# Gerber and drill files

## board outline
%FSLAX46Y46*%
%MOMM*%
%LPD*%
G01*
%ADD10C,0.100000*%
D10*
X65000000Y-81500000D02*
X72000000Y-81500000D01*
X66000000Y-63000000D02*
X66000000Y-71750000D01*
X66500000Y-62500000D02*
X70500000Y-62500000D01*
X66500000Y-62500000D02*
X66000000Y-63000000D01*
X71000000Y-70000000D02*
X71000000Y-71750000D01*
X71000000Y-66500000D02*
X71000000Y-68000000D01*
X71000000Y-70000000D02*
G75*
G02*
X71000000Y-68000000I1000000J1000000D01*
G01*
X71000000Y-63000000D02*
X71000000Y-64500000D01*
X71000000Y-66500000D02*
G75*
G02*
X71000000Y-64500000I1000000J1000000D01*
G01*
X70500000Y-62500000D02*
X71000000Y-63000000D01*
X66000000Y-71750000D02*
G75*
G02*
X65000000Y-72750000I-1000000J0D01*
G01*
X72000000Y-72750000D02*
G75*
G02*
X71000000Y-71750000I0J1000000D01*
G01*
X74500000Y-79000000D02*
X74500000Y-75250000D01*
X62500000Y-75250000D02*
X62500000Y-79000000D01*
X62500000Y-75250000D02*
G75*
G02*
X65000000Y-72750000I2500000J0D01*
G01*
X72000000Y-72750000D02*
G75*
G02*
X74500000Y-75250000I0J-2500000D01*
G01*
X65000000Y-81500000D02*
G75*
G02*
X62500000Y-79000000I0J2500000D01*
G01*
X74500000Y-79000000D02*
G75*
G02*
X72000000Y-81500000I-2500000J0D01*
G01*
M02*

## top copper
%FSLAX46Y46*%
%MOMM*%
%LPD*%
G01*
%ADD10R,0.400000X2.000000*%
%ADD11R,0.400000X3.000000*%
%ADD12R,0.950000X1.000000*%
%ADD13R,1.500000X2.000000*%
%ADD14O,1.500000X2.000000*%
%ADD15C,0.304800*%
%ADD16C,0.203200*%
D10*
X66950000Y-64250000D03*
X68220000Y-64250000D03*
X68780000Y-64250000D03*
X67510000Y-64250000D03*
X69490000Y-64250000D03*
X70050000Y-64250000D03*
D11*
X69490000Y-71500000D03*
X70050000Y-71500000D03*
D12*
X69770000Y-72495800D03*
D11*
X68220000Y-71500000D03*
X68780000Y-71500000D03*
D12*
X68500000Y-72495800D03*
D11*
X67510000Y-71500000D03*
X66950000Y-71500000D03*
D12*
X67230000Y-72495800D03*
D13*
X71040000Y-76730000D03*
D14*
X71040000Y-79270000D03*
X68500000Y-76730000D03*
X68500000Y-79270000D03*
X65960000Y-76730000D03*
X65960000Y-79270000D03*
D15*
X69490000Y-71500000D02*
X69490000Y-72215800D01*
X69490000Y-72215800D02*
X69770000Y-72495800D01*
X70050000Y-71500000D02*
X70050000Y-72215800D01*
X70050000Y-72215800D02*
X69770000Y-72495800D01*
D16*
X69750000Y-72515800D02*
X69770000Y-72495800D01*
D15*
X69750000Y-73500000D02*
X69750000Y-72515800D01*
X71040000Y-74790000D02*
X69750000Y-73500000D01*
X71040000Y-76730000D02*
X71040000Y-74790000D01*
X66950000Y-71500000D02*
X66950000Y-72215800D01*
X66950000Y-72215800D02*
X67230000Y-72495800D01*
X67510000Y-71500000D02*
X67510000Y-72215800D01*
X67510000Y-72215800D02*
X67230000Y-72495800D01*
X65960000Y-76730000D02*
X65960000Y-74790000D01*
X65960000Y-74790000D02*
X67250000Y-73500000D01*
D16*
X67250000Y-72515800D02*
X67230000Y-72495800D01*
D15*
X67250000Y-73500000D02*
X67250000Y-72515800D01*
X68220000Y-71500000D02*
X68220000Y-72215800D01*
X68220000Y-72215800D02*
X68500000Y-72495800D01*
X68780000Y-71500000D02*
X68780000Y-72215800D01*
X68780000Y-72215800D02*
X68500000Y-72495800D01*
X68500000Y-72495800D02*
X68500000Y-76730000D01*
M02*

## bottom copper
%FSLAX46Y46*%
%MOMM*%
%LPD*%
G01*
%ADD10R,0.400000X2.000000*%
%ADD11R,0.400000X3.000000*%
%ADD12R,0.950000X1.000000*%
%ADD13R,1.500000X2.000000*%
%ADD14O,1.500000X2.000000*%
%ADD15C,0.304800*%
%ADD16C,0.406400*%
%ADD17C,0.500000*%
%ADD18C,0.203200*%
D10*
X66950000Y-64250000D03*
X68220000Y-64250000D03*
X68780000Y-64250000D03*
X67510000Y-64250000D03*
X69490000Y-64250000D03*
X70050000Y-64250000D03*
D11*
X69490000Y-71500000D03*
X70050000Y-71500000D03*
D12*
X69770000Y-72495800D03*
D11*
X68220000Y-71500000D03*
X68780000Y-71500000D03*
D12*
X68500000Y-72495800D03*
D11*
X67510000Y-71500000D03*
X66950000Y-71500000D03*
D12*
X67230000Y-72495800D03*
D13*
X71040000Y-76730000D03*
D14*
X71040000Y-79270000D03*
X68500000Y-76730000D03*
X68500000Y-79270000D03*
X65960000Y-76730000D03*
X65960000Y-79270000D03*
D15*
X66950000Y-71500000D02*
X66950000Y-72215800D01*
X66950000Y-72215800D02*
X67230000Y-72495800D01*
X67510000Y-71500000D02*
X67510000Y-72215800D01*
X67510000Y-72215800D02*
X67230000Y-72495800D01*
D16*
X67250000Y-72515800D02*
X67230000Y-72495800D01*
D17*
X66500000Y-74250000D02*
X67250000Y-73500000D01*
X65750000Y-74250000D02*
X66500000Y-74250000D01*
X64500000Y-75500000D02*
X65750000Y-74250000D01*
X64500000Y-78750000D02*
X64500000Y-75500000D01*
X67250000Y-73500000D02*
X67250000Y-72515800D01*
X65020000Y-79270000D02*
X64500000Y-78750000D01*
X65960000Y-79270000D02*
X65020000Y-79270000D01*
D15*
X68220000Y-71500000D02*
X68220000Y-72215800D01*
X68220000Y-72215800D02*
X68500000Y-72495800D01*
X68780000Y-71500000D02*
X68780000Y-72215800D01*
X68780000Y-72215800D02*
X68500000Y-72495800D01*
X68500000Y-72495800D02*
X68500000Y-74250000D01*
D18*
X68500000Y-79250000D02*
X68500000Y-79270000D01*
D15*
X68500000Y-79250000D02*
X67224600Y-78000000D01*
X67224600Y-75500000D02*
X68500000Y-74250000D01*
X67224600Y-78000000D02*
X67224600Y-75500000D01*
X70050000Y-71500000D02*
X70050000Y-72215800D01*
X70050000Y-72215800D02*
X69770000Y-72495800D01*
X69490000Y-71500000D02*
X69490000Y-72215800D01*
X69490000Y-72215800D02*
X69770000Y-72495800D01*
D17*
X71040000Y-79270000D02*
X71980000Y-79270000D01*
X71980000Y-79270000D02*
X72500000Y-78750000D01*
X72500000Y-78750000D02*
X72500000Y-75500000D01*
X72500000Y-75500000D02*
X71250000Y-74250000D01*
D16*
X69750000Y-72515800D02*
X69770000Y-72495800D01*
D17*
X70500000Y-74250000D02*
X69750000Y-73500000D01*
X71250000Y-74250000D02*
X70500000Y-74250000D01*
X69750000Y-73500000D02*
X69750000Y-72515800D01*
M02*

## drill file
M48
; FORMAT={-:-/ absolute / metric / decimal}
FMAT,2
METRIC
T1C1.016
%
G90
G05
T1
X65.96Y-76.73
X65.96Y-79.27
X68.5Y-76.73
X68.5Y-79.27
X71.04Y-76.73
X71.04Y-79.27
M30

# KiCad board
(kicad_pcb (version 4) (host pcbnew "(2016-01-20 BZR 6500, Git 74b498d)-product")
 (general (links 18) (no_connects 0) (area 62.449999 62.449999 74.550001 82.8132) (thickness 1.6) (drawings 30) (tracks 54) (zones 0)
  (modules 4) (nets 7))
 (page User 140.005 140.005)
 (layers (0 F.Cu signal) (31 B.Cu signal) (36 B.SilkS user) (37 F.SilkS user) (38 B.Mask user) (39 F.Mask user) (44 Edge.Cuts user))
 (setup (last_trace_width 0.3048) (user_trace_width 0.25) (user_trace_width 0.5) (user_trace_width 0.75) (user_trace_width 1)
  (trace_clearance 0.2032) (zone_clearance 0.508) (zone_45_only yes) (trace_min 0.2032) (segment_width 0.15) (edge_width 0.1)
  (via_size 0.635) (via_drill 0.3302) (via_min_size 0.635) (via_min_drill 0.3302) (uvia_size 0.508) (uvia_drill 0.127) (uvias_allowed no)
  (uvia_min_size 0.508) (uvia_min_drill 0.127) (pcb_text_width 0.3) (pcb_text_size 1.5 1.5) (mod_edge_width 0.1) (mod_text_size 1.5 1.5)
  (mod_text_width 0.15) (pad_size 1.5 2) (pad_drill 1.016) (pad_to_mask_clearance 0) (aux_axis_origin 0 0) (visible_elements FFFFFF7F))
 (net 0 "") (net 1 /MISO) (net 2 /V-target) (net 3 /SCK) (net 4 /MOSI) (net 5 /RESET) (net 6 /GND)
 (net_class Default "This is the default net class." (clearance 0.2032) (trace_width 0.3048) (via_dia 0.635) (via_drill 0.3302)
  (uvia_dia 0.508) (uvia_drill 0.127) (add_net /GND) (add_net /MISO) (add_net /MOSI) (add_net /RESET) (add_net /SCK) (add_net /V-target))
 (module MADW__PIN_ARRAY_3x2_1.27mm (layer F.Cu) (at 68.5 68) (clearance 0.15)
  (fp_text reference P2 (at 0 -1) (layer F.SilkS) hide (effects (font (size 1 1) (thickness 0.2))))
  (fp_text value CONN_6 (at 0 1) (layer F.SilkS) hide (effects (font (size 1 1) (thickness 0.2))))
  (pad ~ smd rect (at -1.55 -3.75) (size 0.4 2) (layers F.Cu F.Mask))
  (pad ~ smd rect (at -0.28 -3.75) (size 0.4 2) (layers F.Cu F.Mask))
  (pad ~ smd rect (at 0.28 -3.75) (size 0.4 2) (layers F.Cu F.Mask))
  (pad ~ smd rect (at -0.99 -3.75) (size 0.4 2) (layers F.Cu F.Mask))
  (pad ~ smd rect (at 0.99 -3.75) (size 0.4 2) (layers F.Cu F.Mask))
  (pad ~ smd rect (at 1.55 -3.75) (size 0.4 2) (layers F.Cu F.Mask))
  (pad ~ smd rect (at -1.55 -3.75) (size 0.4 2) (layers B.Cu F.Mask))
  (pad ~ smd rect (at -0.28 -3.75) (size 0.4 2) (layers B.Cu F.Mask))
  (pad ~ smd rect (at 0.28 -3.75) (size 0.4 2) (layers B.Cu F.Mask))
  (pad ~ smd rect (at -0.99 -3.75) (size 0.4 2) (layers B.Cu F.Mask))
  (pad ~ smd rect (at 0.99 -3.75) (size 0.4 2) (layers B.Cu F.Mask))
  (pad ~ smd rect (at 1.55 -3.75) (size 0.4 2) (layers B.Cu F.Mask))
  (pad 1 smd rect (at 0.99 3.5) (size 0.4 3) (layers F.Cu F.Mask) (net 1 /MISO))
  (pad 1 smd rect (at 1.55 3.5) (size 0.4 3) (layers F.Cu F.Mask) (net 1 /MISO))
  (pad 1 smd rect (at 1.27 4.4958) (size 0.95 1) (layers F.Cu F.Mask) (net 1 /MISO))
  (pad 2 smd rect (at 0.99 3.5) (size 0.4 3) (layers B.Cu F.Mask) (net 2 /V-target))
  (pad 2 smd rect (at 1.55 3.5) (size 0.4 3) (layers B.Cu F.Mask) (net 2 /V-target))
  (pad 2 smd rect (at 1.27 4.4958) (size 0.95 1) (layers B.Cu B.Mask) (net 2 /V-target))
  (pad 3 smd rect (at -0.28 3.5) (size 0.4 3) (layers F.Cu F.Mask) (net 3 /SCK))
  (pad 3 smd rect (at 0.28 3.5) (size 0.4 3) (layers F.Cu F.Mask) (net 3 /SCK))
  (pad 3 smd rect (at 0 4.4958) (size 0.95 1) (layers F.Cu F.Mask) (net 3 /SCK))
  (pad 4 smd rect (at -0.28 3.5) (size 0.4 3) (layers B.Cu F.Mask) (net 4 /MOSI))
  (pad 4 smd rect (at 0.28 3.5) (size 0.4 3) (layers B.Cu F.Mask) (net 4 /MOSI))
  (pad 4 smd rect (at 0 4.4958) (size 0.95 1) (layers B.Cu B.Mask) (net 4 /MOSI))
  (pad 5 smd rect (at -0.99 3.5) (size 0.4 3) (layers F.Cu F.Mask) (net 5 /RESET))
  (pad 5 smd rect (at -1.55 3.5) (size 0.4 3) (layers F.Cu F.Mask) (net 5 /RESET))
  (pad 5 smd rect (at -1.27 4.4958) (size 0.95 1) (layers F.Cu F.Mask) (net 5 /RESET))
  (pad 6 smd rect (at -0.99 3.5) (size 0.4 3) (layers B.Cu F.Mask) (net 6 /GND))
  (pad 6 smd rect (at -1.55 3.5) (size 0.4 3) (layers B.Cu F.Mask) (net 6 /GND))
  (pad 6 smd rect (at -1.27 4.4958) (size 0.95 1) (layers B.Cu B.Mask) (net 6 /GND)))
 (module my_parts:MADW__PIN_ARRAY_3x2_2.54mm (layer F.Cu) (at 68.5 78)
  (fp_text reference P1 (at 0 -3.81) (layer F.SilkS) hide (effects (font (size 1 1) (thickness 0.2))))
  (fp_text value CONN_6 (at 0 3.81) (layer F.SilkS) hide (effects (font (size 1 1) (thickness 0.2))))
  (pad 1 thru_hole rect (at 2.54 -1.27) (size 1.5 2) (drill 1.016) (layers *.Cu *.Mask F.SilkS) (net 1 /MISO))
  (pad 2 thru_hole oval (at 2.54 1.27) (size 1.5 2) (drill 1.016) (layers *.Cu *.Mask F.SilkS) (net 2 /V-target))
  (pad 3 thru_hole oval (at 0 -1.27) (size 1.5 2) (drill 1.016) (layers *.Cu *.Mask F.SilkS) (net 3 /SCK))
  (pad 4 thru_hole oval (at 0 1.27) (size 1.5 2) (drill 1.016) (layers *.Cu *.Mask F.SilkS) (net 4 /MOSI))
  (pad 5 thru_hole oval (at -2.54 -1.27) (size 1.5 2) (drill 1.016) (layers *.Cu *.Mask F.SilkS) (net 5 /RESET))
  (pad 6 thru_hole oval (at -2.54 1.27) (size 1.5 2) (drill 1.016) (layers *.Cu *.Mask F.SilkS) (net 6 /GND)))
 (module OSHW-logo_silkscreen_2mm (layer F.Cu) (at 71.95 74.2)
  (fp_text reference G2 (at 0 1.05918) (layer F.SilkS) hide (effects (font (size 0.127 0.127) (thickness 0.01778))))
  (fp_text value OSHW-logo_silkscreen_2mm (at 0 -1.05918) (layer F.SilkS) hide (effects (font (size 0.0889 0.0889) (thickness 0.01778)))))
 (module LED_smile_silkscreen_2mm (layer F.Cu) (at 64.75 74.25)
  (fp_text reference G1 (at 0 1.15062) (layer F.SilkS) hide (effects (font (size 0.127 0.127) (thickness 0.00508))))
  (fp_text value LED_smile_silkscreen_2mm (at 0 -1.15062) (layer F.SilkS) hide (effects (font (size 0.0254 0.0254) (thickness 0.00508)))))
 (gr_line (start 65 81.5) (end 72 81.5) (layer Edge.Cuts) (width 0.1))
 (gr_line (start 66 63) (end 66 71.75) (angle 90) (layer Edge.Cuts) (width 0.1))
 (gr_line (start 66.5 62.5) (end 70.5 62.5) (angle 90) (layer Edge.Cuts) (width 0.1))
 (gr_line (start 66.5 62.5) (end 66 63) (angle 90) (layer Edge.Cuts) (width 0.1))
 (gr_line (start 71 70) (end 71 71.75) (angle 90) (layer Edge.Cuts) (width 0.1))
 (gr_line (start 71 66.5) (end 71 68) (angle 90) (layer Edge.Cuts) (width 0.1))
 (gr_arc (start 72 69) (end 71 70) (angle 90) (layer Edge.Cuts) (width 0.1))
 (gr_line (start 71 63) (end 71 64.5) (angle 90) (layer Edge.Cuts) (width 0.1))
 (gr_arc (start 72 65.5) (end 71 66.5) (angle 90) (layer Edge.Cuts) (width 0.1))
 (gr_line (start 70.5 62.5) (end 71 63) (angle 90) (layer Edge.Cuts) (width 0.1))
 (gr_arc (start 65 71.75) (end 66 71.75) (angle 90) (layer Edge.Cuts) (width 0.1))
 (gr_arc (start 72 71.75) (end 72 72.75) (angle 90) (layer Edge.Cuts) (width 0.1))
 (gr_line (start 74.5 79) (end 74.5 75.25) (angle 90) (layer Edge.Cuts) (width 0.1))
 (gr_line (start 62.5 75.25) (end 62.5 79) (angle 90) (layer Edge.Cuts) (width 0.1))
 (gr_arc (start 65 75.25) (end 62.5 75.25) (angle 90) (layer Edge.Cuts) (width 0.1))
 (gr_arc (start 72 75.25) (end 72 72.75) (angle 90) (layer Edge.Cuts) (width 0.1))
 (gr_arc (start 65 79) (end 65 81.5) (angle 90) (layer Edge.Cuts) (width 0.1))
 (gr_arc (start 72 79) (end 74.5 79) (angle 90) (layer Edge.Cuts) (width 0.1))
 (segment (start 66.95 71.5) (end 66.95 72.2158) (width 0.3048) (layer B.Cu) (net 6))
 (segment (start 66.95 72.2158) (end 67.23 72.4958) (width 0.3048) (layer B.Cu) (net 6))
 (segment (start 67.51 71.5) (end 67.51 72.2158) (width 0.3048) (layer B.Cu) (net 6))
 (segment (start 67.51 72.2158) (end 67.23 72.4958) (width 0.3048) (layer B.Cu) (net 6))
 (segment (start 67.25 72.5158) (end 67.23 72.4958) (width 0.4064) (layer B.Cu) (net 6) (status 30))
 (segment (start 66.5 74.25) (end 67.25 73.5) (width 0.5) (layer B.Cu) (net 6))
 (segment (start 65.75 74.25) (end 66.5 74.25) (width 0.5) (layer B.Cu) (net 6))
 (segment (start 64.5 75.5) (end 65.75 74.25) (width 0.5) (layer B.Cu) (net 6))
 (segment (start 64.5 78.75) (end 64.5 75.5) (width 0.5) (layer B.Cu) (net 6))
 (segment (start 67.25 73.5) (end 67.25 72.5158) (width 0.5) (layer B.Cu) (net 6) (status 20))
 (segment (start 65.02 79.27) (end 64.5 78.75) (width 0.5) (layer B.Cu) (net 6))
 (segment (start 65.96 79.27) (end 65.02 79.27) (width 0.5) (layer B.Cu) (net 6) (status 10))
 (segment (start 69.49 71.5) (end 69.49 72.2158) (width 0.3048) (layer F.Cu) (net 1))
 (segment (start 69.49 72.2158) (end 69.77 72.4958) (width 0.3048) (layer F.Cu) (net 1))
 (segment (start 70.05 71.5) (end 70.05 72.2158) (width 0.3048) (layer F.Cu) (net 1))
 (segment (start 70.05 72.2158) (end 69.77 72.4958) (width 0.3048) (layer F.Cu) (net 1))
 (segment (start 69.75 72.5158) (end 69.77 72.4958) (width 0.2032) (layer F.Cu) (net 1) (status 30))
 (segment (start 69.75 73.5) (end 69.75 72.5158) (width 0.3048) (layer F.Cu) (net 1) (status 20))
 (segment (start 71.04 74.79) (end 69.75 73.5) (width 0.3048) (layer F.Cu) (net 1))
 (segment (start 71.04 76.73) (end 71.04 74.79) (width 0.3048) (layer F.Cu) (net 1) (status 10))
 (segment (start 68.22 71.5) (end 68.22 72.2158) (width 0.3048) (layer B.Cu) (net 4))
 (segment (start 68.22 72.2158) (end 68.5 72.4958) (width 0.3048) (layer B.Cu) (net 4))
 (segment (start 68.78 71.5) (end 68.78 72.2158) (width 0.3048) (layer B.Cu) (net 4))
 (segment (start 68.78 72.2158) (end 68.5 72.4958) (width 0.3048) (layer B.Cu) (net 4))
 (segment (start 68.5 72.4958) (end 68.5 74.25) (width 0.3048) (layer B.Cu) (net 4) (status 10))
 (segment (start 68.5 79.25) (end 68.5 79.27) (width 0.2032) (layer B.Cu) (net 4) (status 30))
 (segment (start 68.5 79.25) (end 67.2246 78) (width 0.3048) (layer B.Cu) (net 4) (status 10))
 (segment (start 67.2246 75.5) (end 68.5 74.25) (width 0.3048) (layer B.Cu) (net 4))
 (segment (start 67.2246 78) (end 67.2246 75.5) (width 0.3048) (layer B.Cu) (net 4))
 (segment (start 66.95 71.5) (end 66.95 72.2158) (width 0.3048) (layer F.Cu) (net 5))
 (segment (start 66.95 72.2158) (end 67.23 72.4958) (width 0.3048) (layer F.Cu) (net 5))
 (segment (start 67.51 71.5) (end 67.51 72.2158) (width 0.3048) (layer F.Cu) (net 5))
 (segment (start 67.51 72.2158) (end 67.23 72.4958) (width 0.3048) (layer F.Cu) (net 5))
 (segment (start 65.96 76.73) (end 65.96 74.79) (width 0.3048) (layer F.Cu) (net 5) (status 10))
 (segment (start 65.96 74.79) (end 67.25 73.5) (width 0.3048) (layer F.Cu) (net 5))
 (segment (start 67.25 72.5158) (end 67.23 72.4958) (width 0.2032) (layer F.Cu) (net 5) (status 30))
 (segment (start 67.25 73.5) (end 67.25 72.5158) (width 0.3048) (layer F.Cu) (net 5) (status 20))
 (segment (start 68.22 71.5) (end 68.22 72.2158) (width 0.3048) (layer F.Cu) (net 3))
 (segment (start 68.22 72.2158) (end 68.5 72.4958) (width 0.3048) (layer F.Cu) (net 3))
 (segment (start 68.78 71.5) (end 68.78 72.2158) (width 0.3048) (layer F.Cu) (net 3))
 (segment (start 68.78 72.2158) (end 68.5 72.4958) (width 0.3048) (layer F.Cu) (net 3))
 (segment (start 68.5 72.4958) (end 68.5 76.73) (width 0.3048) (layer F.Cu) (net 3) (status 30))
 (segment (start 70.05 71.5) (end 70.05 72.2158) (width 0.3048) (layer B.Cu) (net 2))
 (segment (start 70.05 72.2158) (end 69.77 72.4958) (width 0.3048) (layer B.Cu) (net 2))
 (segment (start 69.49 71.5) (end 69.49 72.2158) (width 0.3048) (layer B.Cu) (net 2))
 (segment (start 69.49 72.2158) (end 69.77 72.4958) (width 0.3048) (layer B.Cu) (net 2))
 (segment (start 71.04 79.27) (end 71.98 79.27) (width 0.5) (layer B.Cu) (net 2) (status 10))
 (segment (start 71.98 79.27) (end 72.5 78.75) (width 0.5) (layer B.Cu) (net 2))
 (segment (start 72.5 78.75) (end 72.5 75.5) (width 0.5) (layer B.Cu) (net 2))
 (segment (start 72.5 75.5) (end 71.25 74.25) (width 0.5) (layer B.Cu) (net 2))
 (segment (start 69.75 72.5158) (end 69.77 72.4958) (width 0.4064) (layer B.Cu) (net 2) (status 30))
 (segment (start 70.5 74.25) (end 69.75 73.5) (width 0.5) (layer B.Cu) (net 2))
 (segment (start 71.25 74.25) (end 70.5 74.25) (width 0.5) (layer B.Cu) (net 2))
 (segment (start 69.75 73.5) (end 69.75 72.5158) (width 0.5) (layer B.Cu) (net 2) (status 20))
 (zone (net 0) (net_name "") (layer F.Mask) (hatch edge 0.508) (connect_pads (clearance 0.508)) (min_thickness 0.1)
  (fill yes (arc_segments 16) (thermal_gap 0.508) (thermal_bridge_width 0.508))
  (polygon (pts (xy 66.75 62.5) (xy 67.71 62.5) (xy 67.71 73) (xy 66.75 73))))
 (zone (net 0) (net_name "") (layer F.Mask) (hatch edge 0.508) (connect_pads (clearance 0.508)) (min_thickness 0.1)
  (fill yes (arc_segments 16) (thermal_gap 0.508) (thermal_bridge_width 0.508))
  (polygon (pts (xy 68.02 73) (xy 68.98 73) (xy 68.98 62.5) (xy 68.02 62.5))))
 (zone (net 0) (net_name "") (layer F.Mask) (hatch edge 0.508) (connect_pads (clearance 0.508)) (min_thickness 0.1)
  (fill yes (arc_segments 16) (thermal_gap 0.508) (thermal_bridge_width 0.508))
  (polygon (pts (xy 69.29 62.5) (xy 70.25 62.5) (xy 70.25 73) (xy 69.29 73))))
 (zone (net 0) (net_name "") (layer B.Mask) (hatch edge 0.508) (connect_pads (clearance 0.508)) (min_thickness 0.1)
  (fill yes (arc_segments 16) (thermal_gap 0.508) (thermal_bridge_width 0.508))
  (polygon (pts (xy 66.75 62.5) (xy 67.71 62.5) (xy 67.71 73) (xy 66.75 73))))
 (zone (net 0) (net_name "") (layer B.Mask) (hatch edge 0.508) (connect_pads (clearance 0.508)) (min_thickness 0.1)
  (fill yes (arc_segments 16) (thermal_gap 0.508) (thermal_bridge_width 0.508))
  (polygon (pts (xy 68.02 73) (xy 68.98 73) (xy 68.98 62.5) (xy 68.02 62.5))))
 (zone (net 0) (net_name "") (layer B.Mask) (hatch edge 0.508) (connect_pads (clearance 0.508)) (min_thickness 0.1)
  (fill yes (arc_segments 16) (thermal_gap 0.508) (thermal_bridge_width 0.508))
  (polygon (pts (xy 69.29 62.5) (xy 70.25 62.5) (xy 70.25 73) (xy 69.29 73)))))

